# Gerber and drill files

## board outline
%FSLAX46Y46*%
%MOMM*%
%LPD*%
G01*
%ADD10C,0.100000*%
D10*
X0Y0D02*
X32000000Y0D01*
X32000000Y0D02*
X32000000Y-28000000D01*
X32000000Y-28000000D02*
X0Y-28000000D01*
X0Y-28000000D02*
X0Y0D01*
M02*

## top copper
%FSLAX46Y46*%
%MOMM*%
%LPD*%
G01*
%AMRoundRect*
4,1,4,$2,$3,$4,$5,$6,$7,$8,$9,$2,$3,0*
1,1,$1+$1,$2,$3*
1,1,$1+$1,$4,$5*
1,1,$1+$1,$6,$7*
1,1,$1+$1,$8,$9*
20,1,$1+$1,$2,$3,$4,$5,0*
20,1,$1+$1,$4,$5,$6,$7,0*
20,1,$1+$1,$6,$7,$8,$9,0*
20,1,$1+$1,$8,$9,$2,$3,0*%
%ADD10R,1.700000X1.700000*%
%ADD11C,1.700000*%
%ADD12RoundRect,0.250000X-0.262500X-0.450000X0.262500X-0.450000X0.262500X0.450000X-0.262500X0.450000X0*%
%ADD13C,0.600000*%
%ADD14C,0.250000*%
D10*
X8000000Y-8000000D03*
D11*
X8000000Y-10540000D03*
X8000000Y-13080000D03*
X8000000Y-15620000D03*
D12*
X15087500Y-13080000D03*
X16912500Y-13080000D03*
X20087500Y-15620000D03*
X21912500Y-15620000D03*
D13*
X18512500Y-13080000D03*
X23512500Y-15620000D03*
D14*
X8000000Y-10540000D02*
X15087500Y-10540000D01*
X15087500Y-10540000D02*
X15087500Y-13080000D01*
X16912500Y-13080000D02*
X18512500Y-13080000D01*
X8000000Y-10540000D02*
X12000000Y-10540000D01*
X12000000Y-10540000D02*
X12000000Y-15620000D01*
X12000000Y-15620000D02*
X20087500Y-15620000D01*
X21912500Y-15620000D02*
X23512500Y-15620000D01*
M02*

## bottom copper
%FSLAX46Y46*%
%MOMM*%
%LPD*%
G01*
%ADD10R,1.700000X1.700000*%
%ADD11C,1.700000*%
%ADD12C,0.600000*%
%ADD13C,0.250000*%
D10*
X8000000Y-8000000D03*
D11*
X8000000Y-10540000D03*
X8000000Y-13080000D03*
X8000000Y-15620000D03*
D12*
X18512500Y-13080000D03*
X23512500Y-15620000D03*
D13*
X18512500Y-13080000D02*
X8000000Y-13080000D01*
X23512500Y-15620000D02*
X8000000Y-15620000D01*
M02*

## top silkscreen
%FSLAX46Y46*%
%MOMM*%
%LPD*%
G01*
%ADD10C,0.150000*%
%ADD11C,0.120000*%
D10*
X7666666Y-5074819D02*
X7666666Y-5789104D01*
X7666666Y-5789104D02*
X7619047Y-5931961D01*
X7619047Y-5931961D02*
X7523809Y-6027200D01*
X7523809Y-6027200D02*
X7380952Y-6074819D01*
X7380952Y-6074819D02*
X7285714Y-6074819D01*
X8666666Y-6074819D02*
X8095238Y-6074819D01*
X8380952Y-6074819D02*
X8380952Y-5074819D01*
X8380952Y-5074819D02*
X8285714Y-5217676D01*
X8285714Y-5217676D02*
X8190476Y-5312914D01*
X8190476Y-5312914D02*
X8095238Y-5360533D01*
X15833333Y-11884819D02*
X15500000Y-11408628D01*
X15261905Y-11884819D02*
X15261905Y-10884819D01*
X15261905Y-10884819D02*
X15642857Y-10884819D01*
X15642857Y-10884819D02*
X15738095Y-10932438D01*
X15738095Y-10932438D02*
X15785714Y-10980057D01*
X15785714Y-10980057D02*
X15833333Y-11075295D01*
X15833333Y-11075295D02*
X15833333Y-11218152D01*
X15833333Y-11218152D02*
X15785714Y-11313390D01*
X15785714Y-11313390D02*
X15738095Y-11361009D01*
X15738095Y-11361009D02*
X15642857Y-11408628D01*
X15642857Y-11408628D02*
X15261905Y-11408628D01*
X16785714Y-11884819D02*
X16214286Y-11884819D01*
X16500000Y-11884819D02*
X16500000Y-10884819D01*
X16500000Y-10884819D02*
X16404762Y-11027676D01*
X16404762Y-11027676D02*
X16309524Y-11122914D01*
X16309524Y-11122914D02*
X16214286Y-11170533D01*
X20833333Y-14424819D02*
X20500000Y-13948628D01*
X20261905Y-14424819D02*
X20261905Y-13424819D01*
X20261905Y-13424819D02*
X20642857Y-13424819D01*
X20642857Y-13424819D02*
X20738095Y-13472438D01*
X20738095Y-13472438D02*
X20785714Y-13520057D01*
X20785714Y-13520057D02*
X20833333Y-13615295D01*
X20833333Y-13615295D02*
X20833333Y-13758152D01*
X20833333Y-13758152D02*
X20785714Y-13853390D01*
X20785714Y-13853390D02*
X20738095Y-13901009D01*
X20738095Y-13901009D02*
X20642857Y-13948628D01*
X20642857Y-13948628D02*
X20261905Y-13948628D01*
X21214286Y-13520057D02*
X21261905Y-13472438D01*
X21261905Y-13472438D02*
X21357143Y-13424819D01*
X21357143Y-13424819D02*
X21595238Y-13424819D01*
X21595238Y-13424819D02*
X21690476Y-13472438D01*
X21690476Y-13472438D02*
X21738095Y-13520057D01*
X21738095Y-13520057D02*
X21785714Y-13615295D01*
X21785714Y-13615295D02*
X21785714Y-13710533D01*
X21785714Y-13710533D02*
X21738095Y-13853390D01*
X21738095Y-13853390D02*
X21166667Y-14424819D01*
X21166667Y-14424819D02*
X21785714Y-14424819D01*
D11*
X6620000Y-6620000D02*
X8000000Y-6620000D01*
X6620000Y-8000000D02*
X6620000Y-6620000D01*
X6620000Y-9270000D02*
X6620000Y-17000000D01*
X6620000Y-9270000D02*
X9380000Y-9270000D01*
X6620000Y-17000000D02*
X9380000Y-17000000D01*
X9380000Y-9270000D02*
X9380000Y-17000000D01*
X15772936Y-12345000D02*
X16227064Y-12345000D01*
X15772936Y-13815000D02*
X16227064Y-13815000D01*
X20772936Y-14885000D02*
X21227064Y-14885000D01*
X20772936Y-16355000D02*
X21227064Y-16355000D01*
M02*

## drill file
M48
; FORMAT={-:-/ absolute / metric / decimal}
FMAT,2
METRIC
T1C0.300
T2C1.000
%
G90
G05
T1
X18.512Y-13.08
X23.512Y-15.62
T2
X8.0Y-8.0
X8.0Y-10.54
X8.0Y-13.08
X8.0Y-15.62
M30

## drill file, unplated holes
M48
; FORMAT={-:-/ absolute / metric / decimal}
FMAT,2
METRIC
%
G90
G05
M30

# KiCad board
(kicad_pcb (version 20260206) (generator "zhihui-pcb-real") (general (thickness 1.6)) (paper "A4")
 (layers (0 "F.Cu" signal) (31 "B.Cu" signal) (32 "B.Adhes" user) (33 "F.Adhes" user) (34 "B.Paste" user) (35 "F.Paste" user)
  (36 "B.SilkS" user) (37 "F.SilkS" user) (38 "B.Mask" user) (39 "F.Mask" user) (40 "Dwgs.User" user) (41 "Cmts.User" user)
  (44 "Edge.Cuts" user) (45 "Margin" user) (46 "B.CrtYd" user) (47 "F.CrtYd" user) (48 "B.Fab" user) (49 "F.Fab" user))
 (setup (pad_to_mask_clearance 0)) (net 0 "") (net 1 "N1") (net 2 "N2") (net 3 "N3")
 (gr_line (start 0 0) (end 32 0) (stroke (width 0.1) (type default)) (layer "Edge.Cuts"))
 (gr_line (start 32 0) (end 32 28) (stroke (width 0.1) (type default)) (layer "Edge.Cuts"))
 (gr_line (start 32 28) (end 0 28) (stroke (width 0.1) (type default)) (layer "Edge.Cuts"))
 (gr_line (start 0 28) (end 0 0) (stroke (width 0.1) (type default)) (layer "Edge.Cuts"))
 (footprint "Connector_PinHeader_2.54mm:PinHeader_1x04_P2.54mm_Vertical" (layer "F.Cu")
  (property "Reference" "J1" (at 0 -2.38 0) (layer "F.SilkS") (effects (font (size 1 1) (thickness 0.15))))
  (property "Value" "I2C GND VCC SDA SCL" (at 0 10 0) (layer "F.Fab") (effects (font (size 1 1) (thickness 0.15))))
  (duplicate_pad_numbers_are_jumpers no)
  (fp_line (start -1.38 -1.38) (end 0 -1.38) (stroke (width 0.12) (type solid)) (layer "F.SilkS"))
  (fp_line (start -1.38 0) (end -1.38 -1.38) (stroke (width 0.12) (type solid)) (layer "F.SilkS"))
  (fp_line (start -1.38 1.27) (end -1.38 9) (stroke (width 0.12) (type solid)) (layer "F.SilkS"))
  (fp_line (start -1.38 1.27) (end 1.38 1.27) (stroke (width 0.12) (type solid)) (layer "F.SilkS"))
  (fp_line (start -1.38 9) (end 1.38 9) (stroke (width 0.12) (type solid)) (layer "F.SilkS"))
  (fp_line (start 1.38 1.27) (end 1.38 9) (stroke (width 0.12) (type solid)) (layer "F.SilkS"))
  (pad "1" thru_hole rect (at 0 0) (size 1.7 1.7) (drill 1) (layers "*.Cu" "*.Mask") (remove_unused_layers no))
  (pad "2" thru_hole circle (at 0 2.54) (size 1.7 1.7) (drill 1) (layers "*.Cu" "*.Mask") (remove_unused_layers no) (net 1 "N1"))
  (pad "3" thru_hole circle (at 0 5.08) (size 1.7 1.7) (drill 1) (layers "*.Cu" "*.Mask") (remove_unused_layers no) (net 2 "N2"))
  (pad "4" thru_hole circle (at 0 7.62) (size 1.7 1.7) (drill 1) (layers "*.Cu" "*.Mask") (remove_unused_layers no) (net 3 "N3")) (at 8 8 0))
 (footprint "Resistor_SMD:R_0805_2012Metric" (layer "F.Cu")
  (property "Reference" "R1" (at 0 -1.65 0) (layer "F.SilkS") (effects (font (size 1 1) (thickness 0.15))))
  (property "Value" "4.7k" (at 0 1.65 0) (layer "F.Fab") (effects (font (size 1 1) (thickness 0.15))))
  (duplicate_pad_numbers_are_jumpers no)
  (fp_line (start -0.227064 -0.735) (end 0.227064 -0.735) (stroke (width 0.12) (type solid)) (layer "F.SilkS"))
  (fp_line (start -0.227064 0.735) (end 0.227064 0.735) (stroke (width 0.12) (type solid)) (layer "F.SilkS"))
  (pad "1" smd roundrect (at -0.9125 0) (size 1.025 1.4) (layers "F.Cu" "F.Mask" "F.Paste") (roundrect_rratio 0.243902) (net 1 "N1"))
  (pad "2" smd roundrect (at 0.9125 0) (size 1.025 1.4) (layers "F.Cu" "F.Mask" "F.Paste") (roundrect_rratio 0.243902) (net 2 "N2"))
  (at 16 13.08 0))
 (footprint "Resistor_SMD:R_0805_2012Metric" (layer "F.Cu")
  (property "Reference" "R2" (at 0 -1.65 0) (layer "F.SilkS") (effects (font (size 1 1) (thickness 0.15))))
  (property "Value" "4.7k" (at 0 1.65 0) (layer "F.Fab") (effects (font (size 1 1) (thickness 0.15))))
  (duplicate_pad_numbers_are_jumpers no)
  (fp_line (start -0.227064 -0.735) (end 0.227064 -0.735) (stroke (width 0.12) (type solid)) (layer "F.SilkS"))
  (fp_line (start -0.227064 0.735) (end 0.227064 0.735) (stroke (width 0.12) (type solid)) (layer "F.SilkS"))
  (pad "1" smd roundrect (at -0.9125 0) (size 1.025 1.4) (layers "F.Cu" "F.Mask" "F.Paste") (roundrect_rratio 0.243902) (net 1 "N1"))
  (pad "2" smd roundrect (at 0.9125 0) (size 1.025 1.4) (layers "F.Cu" "F.Mask" "F.Paste") (roundrect_rratio 0.243902) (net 3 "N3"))
  (at 21 15.62 0))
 (segment (start 8 10.54) (end 15.0875 10.54) (width 0.25) (layer "F.Cu") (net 1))
 (segment (start 15.0875 10.54) (end 15.0875 13.08) (width 0.25) (layer "F.Cu") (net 1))
 (segment (start 16.9125 13.08) (end 18.5125 13.08) (width 0.25) (layer "F.Cu") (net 2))
 (segment (start 18.5125 13.08) (end 8 13.08) (width 0.25) (layer "B.Cu") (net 2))
 (segment (start 8 10.54) (end 12 10.54) (width 0.25) (layer "F.Cu") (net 1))
 (segment (start 12 10.54) (end 12 15.62) (width 0.25) (layer "F.Cu") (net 1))
 (segment (start 12 15.62) (end 20.0875 15.62) (width 0.25) (layer "F.Cu") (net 1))
 (segment (start 21.9125 15.62) (end 23.5125 15.62) (width 0.25) (layer "F.Cu") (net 3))
 (segment (start 23.5125 15.62) (end 8 15.62) (width 0.25) (layer "B.Cu") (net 3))
 (via (at 18.5125 13.08) (size 0.6) (drill 0.3) (layers "F.Cu" "B.Cu") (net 2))
 (via (at 23.5125 15.62) (size 0.6) (drill 0.3) (layers "F.Cu" "B.Cu") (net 3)))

